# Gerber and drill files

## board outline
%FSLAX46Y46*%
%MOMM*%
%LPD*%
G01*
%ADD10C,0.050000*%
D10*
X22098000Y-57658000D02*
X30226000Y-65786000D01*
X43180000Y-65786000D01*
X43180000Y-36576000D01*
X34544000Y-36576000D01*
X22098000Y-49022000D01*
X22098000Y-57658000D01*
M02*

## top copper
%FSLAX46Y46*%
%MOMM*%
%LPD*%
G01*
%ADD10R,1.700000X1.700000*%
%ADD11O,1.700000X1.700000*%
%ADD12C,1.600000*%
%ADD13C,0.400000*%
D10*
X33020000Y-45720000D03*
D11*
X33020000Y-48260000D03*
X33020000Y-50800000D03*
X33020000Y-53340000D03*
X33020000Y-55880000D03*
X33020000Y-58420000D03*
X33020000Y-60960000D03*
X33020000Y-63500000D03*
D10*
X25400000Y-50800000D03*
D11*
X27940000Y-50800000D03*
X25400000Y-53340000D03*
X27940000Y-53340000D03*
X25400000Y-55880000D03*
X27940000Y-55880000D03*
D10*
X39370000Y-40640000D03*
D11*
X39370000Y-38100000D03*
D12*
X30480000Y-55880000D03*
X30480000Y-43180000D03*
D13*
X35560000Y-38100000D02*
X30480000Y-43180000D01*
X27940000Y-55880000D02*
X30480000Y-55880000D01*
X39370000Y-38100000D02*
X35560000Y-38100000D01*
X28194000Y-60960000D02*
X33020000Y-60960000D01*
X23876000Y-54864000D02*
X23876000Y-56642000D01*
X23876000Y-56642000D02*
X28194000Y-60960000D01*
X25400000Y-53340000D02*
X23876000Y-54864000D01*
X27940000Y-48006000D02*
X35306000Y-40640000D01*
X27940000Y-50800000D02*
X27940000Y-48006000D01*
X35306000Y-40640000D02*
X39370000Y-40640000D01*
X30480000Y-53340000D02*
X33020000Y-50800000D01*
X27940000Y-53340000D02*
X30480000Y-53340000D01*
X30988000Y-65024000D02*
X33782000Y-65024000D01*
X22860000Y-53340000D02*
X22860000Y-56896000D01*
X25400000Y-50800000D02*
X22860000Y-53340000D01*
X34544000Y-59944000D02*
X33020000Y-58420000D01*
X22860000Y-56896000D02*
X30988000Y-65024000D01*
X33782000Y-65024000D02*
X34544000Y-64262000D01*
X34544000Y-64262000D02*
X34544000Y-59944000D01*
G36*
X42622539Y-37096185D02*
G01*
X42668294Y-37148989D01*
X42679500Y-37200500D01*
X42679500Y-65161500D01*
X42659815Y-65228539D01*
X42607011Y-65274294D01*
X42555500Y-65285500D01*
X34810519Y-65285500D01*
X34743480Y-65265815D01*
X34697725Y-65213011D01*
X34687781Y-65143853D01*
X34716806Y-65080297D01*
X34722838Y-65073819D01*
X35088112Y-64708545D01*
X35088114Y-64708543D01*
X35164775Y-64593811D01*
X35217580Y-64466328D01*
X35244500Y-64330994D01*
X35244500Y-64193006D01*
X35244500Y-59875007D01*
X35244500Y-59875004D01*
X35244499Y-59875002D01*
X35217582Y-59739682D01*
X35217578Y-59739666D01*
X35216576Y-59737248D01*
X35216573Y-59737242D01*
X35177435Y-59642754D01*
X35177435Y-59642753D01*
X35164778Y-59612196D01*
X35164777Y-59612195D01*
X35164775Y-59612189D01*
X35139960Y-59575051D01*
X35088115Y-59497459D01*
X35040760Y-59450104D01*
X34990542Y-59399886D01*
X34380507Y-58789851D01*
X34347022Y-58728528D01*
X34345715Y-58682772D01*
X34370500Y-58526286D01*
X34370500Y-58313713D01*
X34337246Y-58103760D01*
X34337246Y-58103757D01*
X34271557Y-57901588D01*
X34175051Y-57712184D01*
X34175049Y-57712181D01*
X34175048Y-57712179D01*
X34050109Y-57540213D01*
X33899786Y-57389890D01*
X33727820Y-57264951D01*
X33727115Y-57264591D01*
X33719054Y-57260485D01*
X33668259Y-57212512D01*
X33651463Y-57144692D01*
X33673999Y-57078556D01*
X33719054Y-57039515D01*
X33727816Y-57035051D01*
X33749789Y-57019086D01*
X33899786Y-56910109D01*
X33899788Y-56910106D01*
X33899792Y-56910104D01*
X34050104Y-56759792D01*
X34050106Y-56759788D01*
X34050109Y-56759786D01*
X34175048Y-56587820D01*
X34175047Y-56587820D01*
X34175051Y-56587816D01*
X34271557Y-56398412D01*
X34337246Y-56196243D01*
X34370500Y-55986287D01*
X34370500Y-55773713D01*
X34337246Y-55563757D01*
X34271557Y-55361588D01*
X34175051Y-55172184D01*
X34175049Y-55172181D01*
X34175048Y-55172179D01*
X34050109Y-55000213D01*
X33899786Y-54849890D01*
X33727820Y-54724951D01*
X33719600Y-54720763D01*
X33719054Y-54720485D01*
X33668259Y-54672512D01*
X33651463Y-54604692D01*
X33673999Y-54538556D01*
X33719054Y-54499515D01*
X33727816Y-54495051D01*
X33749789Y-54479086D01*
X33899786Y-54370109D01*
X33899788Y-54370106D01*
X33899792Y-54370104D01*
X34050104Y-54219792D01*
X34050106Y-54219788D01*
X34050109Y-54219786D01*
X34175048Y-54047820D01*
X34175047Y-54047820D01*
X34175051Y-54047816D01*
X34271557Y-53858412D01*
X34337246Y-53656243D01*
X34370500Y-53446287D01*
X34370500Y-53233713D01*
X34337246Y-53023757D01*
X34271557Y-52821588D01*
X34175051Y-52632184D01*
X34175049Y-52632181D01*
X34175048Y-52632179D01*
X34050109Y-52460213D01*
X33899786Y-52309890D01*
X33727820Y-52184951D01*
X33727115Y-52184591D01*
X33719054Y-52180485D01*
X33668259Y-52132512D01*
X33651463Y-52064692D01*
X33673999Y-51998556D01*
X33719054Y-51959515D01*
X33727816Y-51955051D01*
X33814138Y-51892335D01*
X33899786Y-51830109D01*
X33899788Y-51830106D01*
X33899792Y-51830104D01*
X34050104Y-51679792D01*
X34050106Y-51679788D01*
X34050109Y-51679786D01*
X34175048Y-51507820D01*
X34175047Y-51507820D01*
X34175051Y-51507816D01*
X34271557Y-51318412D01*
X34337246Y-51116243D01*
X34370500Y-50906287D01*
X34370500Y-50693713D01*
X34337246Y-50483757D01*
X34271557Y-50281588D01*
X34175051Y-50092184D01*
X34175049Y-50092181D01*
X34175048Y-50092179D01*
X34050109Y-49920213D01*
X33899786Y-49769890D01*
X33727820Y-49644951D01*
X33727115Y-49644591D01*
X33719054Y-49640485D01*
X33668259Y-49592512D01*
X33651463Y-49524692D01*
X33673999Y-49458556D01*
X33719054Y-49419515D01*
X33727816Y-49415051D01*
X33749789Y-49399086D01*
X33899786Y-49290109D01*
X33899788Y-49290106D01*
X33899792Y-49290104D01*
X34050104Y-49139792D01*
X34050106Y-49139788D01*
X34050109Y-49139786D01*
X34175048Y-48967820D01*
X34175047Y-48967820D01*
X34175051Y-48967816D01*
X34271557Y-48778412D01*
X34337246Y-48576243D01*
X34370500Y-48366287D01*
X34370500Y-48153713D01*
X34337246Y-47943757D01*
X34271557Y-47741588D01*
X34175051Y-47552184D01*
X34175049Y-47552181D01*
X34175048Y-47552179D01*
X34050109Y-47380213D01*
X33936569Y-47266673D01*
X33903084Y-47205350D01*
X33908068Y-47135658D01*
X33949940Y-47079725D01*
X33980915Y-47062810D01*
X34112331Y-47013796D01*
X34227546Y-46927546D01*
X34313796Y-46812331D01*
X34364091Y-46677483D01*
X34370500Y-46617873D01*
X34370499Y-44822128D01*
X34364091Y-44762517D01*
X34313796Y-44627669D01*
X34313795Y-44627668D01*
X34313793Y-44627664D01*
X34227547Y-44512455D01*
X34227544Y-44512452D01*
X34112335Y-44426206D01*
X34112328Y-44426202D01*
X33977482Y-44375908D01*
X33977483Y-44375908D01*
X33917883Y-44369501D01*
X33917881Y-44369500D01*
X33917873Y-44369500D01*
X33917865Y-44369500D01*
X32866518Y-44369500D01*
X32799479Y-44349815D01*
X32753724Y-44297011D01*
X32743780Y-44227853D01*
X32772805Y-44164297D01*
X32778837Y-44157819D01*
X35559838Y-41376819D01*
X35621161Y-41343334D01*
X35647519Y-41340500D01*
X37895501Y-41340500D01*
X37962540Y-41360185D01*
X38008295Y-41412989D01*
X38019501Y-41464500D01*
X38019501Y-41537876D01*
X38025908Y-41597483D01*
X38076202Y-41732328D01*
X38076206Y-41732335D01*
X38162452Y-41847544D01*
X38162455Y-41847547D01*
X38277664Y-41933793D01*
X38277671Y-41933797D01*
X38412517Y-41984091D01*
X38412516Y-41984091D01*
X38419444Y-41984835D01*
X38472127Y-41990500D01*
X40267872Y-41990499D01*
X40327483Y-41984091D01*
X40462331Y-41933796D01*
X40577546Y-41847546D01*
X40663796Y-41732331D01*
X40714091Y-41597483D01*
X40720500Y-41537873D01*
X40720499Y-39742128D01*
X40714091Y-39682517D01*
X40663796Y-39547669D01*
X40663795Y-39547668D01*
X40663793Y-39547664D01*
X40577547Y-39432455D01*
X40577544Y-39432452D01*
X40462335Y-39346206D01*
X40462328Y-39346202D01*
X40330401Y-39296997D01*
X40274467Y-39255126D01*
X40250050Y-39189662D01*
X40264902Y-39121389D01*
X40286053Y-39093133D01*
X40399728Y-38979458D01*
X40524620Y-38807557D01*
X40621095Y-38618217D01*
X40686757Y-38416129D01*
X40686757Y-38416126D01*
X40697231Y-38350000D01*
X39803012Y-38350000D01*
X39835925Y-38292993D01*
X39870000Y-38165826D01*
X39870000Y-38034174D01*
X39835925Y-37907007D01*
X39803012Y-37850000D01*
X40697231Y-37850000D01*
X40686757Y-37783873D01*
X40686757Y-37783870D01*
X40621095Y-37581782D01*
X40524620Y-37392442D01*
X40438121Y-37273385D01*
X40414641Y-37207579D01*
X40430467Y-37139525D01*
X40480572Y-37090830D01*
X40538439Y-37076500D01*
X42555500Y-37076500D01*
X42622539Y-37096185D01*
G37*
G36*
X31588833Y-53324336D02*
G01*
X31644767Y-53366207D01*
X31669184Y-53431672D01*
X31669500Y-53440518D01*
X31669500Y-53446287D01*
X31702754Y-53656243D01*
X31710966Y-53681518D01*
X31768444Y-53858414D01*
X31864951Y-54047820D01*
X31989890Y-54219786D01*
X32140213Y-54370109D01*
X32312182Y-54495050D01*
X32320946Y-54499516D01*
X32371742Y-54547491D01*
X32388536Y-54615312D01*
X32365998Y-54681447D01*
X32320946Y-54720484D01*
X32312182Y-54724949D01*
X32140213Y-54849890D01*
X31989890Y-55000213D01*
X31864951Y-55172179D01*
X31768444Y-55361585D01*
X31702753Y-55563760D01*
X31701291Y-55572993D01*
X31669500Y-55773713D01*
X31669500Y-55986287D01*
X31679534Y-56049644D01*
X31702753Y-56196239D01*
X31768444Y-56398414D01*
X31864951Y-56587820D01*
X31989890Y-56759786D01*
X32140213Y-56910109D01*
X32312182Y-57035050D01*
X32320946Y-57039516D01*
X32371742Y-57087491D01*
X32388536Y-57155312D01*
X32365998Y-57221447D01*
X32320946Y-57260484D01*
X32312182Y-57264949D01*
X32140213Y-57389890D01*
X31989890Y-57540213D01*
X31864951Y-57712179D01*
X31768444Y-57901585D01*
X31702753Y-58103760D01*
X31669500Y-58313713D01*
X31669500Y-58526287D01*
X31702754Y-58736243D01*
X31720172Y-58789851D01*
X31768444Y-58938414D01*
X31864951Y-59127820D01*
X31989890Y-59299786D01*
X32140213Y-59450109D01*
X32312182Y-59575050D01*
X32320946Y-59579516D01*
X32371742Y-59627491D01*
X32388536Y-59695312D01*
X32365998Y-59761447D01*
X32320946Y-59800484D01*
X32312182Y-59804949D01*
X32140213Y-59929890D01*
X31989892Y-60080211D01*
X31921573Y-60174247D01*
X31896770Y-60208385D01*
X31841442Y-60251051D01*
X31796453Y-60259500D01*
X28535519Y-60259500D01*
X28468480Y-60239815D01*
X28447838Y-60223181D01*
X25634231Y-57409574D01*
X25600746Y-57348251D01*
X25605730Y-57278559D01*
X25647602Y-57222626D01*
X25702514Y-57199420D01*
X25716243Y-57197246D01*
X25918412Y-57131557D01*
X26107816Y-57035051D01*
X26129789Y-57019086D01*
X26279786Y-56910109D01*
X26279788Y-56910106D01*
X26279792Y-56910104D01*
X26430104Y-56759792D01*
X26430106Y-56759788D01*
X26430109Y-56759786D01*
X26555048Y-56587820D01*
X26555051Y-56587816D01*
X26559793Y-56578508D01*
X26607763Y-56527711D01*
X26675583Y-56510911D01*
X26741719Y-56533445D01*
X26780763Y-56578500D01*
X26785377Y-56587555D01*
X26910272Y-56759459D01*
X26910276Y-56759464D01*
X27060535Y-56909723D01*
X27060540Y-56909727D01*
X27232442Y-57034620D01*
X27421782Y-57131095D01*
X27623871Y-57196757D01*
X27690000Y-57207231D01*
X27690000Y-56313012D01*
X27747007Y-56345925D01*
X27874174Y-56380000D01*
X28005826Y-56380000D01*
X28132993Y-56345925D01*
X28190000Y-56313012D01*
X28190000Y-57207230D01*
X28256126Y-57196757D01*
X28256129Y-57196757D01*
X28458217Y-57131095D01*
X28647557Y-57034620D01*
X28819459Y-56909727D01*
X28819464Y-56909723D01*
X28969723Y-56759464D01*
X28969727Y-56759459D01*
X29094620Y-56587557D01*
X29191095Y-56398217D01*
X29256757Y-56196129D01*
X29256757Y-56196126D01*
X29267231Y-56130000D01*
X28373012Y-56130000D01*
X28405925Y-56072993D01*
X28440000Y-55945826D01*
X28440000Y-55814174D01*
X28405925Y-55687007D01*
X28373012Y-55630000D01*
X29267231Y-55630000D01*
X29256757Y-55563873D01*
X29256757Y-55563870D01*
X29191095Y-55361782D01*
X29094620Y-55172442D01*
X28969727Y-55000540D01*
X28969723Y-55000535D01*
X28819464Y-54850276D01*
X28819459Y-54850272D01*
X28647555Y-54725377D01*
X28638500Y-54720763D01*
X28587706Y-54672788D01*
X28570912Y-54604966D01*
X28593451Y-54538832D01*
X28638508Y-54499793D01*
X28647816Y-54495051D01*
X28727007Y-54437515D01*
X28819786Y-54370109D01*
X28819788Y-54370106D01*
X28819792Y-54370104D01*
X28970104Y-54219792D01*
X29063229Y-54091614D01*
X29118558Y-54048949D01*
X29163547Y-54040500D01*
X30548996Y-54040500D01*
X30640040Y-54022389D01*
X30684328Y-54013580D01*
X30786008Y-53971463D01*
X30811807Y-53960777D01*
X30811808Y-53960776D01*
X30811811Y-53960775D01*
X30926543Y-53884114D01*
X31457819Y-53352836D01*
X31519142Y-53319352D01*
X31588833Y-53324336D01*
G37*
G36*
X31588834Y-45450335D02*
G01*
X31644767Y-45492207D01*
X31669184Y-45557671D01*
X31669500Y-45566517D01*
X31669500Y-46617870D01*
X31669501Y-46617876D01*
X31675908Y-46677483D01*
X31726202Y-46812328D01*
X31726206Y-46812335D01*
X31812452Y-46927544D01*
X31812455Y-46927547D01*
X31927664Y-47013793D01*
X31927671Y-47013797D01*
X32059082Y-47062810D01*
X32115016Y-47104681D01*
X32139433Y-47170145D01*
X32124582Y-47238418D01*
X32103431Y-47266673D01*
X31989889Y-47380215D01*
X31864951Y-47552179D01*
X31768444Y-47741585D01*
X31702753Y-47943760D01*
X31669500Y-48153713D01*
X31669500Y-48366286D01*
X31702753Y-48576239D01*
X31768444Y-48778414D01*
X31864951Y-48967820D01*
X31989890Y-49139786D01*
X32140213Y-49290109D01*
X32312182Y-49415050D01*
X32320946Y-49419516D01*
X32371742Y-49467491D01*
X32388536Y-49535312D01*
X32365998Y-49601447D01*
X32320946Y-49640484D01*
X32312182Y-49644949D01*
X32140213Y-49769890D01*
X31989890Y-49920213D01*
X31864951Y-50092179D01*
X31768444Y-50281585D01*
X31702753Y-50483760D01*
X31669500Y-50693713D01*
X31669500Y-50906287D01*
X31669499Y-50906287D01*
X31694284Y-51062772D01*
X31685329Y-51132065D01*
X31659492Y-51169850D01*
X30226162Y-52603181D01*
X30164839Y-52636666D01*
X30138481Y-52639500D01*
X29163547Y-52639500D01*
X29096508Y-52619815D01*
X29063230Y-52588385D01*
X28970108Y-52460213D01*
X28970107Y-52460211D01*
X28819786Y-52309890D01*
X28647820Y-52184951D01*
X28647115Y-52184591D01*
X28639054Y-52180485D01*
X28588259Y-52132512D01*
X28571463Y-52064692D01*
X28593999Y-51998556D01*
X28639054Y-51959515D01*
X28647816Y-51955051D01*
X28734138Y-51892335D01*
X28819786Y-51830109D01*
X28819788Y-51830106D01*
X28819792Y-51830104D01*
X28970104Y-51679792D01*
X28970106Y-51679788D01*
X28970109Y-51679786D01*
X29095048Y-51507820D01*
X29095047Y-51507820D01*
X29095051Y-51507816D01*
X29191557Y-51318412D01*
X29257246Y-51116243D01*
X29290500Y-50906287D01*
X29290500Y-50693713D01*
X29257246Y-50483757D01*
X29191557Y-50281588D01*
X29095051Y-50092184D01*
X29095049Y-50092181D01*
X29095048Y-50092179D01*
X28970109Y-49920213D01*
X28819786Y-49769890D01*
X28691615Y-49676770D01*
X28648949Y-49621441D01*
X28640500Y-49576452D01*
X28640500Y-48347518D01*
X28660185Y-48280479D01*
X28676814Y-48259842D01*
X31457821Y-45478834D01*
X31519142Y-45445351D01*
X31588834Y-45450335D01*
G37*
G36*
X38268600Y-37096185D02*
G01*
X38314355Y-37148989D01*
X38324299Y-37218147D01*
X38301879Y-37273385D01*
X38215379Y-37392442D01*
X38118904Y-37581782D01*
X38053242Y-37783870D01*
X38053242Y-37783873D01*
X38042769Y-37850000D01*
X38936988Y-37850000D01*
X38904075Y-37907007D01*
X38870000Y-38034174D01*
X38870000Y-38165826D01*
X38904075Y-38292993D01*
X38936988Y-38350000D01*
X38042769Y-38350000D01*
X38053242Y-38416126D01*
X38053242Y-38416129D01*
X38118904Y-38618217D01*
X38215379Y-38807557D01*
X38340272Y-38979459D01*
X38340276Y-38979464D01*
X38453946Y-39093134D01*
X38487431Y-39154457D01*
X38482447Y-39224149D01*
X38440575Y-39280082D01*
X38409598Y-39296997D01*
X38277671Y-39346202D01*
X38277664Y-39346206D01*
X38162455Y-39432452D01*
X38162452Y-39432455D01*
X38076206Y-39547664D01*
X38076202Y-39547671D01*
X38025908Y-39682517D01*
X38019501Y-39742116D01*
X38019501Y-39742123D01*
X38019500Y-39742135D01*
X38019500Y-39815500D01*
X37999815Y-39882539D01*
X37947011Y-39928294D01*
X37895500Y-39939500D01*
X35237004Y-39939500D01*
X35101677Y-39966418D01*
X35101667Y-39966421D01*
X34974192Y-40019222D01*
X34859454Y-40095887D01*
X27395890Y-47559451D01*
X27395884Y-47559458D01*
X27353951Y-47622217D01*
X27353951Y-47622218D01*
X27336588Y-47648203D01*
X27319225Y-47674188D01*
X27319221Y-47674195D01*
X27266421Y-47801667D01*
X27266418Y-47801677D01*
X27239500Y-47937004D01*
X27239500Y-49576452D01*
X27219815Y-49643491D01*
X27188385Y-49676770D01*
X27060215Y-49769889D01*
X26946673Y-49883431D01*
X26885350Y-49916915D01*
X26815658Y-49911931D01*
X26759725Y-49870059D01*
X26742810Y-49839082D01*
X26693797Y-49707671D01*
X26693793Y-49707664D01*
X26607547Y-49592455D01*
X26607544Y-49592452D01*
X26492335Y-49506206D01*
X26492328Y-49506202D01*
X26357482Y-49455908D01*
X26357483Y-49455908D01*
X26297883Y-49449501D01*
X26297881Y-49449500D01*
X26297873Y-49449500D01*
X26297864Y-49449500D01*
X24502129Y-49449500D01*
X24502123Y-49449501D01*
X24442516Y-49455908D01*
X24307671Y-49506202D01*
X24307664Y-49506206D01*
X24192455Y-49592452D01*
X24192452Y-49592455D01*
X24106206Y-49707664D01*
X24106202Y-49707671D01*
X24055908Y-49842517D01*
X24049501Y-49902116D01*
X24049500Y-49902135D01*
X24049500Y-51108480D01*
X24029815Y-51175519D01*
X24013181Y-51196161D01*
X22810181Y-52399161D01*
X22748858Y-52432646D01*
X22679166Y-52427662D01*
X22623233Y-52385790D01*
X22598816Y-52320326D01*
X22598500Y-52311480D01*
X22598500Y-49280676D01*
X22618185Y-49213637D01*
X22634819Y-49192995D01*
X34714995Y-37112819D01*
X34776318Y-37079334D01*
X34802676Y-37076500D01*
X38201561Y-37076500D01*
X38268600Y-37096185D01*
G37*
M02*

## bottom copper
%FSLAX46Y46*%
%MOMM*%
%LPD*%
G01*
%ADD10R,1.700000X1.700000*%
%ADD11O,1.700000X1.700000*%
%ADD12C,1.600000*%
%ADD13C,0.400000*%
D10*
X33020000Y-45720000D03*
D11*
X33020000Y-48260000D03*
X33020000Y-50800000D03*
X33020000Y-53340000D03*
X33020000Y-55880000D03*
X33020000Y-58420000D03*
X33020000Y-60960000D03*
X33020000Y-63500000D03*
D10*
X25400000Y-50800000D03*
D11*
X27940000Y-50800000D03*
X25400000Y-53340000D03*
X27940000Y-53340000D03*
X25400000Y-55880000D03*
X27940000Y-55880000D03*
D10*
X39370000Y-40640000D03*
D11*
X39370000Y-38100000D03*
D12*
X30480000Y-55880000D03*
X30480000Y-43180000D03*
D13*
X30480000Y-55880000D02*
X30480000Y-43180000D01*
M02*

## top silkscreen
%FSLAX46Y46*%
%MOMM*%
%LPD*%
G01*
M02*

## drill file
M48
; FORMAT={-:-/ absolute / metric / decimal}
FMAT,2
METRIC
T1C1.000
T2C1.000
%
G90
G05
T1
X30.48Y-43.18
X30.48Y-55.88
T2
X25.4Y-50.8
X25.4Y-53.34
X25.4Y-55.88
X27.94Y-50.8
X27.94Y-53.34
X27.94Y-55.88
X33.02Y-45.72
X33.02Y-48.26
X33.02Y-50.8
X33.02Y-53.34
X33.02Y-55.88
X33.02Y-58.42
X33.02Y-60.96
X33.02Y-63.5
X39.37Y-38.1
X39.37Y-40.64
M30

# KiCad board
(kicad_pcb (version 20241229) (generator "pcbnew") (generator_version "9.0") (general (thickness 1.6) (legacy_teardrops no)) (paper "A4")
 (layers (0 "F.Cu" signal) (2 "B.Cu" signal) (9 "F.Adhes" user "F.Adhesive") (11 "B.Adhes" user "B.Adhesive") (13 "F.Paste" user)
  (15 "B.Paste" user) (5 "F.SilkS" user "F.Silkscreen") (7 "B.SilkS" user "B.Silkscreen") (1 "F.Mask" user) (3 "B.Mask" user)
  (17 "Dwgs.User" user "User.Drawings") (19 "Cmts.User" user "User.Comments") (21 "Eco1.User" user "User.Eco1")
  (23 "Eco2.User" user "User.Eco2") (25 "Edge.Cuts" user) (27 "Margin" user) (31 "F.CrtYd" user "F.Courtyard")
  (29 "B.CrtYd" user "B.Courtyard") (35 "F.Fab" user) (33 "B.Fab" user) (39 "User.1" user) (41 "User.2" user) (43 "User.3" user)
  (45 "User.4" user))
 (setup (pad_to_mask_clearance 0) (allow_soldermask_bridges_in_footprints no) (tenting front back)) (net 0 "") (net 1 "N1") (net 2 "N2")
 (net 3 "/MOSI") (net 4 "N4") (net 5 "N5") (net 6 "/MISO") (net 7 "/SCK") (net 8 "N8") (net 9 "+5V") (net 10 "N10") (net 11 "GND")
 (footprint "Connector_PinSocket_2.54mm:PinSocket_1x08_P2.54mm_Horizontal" (layer "B.Cu") (at 33.02 45.72 180)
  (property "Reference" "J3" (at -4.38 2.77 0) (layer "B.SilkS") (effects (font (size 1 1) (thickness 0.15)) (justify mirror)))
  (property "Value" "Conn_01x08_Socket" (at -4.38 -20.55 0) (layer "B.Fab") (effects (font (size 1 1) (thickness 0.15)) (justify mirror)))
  (pad "1" thru_hole rect (at 0 0 180) (size 1.7 1.7) (drill 1) (layers "*.Cu" "*.Mask") (remove_unused_layers no) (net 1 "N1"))
  (pad "2" thru_hole oval (at 0 -2.54 180) (size 1.7 1.7) (drill 1) (layers "*.Cu" "*.Mask") (remove_unused_layers no) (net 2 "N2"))
  (pad "3" thru_hole oval (at 0 -5.08 180) (size 1.7 1.7) (drill 1) (layers "*.Cu" "*.Mask") (remove_unused_layers no) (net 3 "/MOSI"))
  (pad "4" thru_hole oval (at 0 -7.62 180) (size 1.7 1.7) (drill 1) (layers "*.Cu" "*.Mask") (remove_unused_layers no) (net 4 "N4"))
  (pad "5" thru_hole oval (at 0 -10.16 180) (size 1.7 1.7) (drill 1) (layers "*.Cu" "*.Mask") (remove_unused_layers no) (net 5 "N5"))
  (pad "6" thru_hole oval (at 0 -12.7 180) (size 1.7 1.7) (drill 1) (layers "*.Cu" "*.Mask") (remove_unused_layers no) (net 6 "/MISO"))
  (pad "7" thru_hole oval (at 0 -15.24 180) (size 1.7 1.7) (drill 1) (layers "*.Cu" "*.Mask") (remove_unused_layers no) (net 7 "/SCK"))
  (pad "8" thru_hole oval (at 0 -17.78 180) (size 1.7 1.7) (drill 1) (layers "*.Cu" "*.Mask") (remove_unused_layers no) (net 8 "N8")))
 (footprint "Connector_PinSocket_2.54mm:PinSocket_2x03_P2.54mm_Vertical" (layer "B.Cu") (at 25.4 50.8 180)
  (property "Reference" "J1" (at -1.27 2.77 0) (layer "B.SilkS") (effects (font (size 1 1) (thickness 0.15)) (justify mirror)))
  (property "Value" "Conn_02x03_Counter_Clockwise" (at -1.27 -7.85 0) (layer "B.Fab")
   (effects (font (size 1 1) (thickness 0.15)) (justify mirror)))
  (pad "1" thru_hole rect (at 0 0 180) (size 1.7 1.7) (drill 1) (layers "*.Cu" "*.Mask") (remove_unused_layers no) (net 6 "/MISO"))
  (pad "2" thru_hole oval (at -2.54 0 180) (size 1.7 1.7) (drill 1) (layers "*.Cu" "*.Mask") (remove_unused_layers no) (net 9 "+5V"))
  (pad "3" thru_hole oval (at 0 -2.54 180) (size 1.7 1.7) (drill 1) (layers "*.Cu" "*.Mask") (remove_unused_layers no) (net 7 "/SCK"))
  (pad "4" thru_hole oval (at -2.54 -2.54 180) (size 1.7 1.7) (drill 1) (layers "*.Cu" "*.Mask") (remove_unused_layers no) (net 3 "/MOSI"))
  (pad "5" thru_hole oval (at 0 -5.08 180) (size 1.7 1.7) (drill 1) (layers "*.Cu" "*.Mask") (remove_unused_layers no) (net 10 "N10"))
  (pad "6" thru_hole oval (at -2.54 -5.08 180) (size 1.7 1.7) (drill 1) (layers "*.Cu" "*.Mask") (remove_unused_layers no) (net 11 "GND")))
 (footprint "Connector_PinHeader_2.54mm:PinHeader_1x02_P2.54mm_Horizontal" (layer "B.Cu") (at 39.37 40.64)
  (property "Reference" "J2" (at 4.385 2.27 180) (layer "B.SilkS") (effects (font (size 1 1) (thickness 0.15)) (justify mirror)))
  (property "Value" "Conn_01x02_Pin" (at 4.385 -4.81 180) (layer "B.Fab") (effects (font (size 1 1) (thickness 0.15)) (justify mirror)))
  (pad "1" thru_hole rect (at 0 0) (size 1.7 1.7) (drill 1) (layers "*.Cu" "*.Mask") (remove_unused_layers no) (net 9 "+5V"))
  (pad "2" thru_hole oval (at 0 -2.54) (size 1.7 1.7) (drill 1) (layers "*.Cu" "*.Mask") (remove_unused_layers no) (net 11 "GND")))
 (gr_poly
  (pts (xy 22.098 57.658) (xy 30.226 65.786) (xy 43.18 65.786) (xy 43.18 36.576) (xy 34.544 36.576) (xy 22.098 49.022))
  (stroke (width 0.05) (type solid)) (fill no) (layer "Edge.Cuts"))
 (segment (start 35.56 38.1) (end 30.48 43.18) (width 0.4) (layer "F.Cu") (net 11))
 (segment (start 27.94 55.88) (end 30.48 55.88) (width 0.4) (layer "F.Cu") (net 11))
 (segment (start 39.37 38.1) (end 35.56 38.1) (width 0.4) (layer "F.Cu") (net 11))
 (via (at 30.48 55.88) (size 1.6) (drill 1) (layers "F.Cu" "B.Cu") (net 11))
 (via (at 30.48 43.18) (size 1.6) (drill 1) (layers "F.Cu" "B.Cu") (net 11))
 (segment (start 30.48 55.88) (end 30.48 43.18) (width 0.4) (layer "B.Cu") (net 11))
 (segment (start 28.194 60.96) (end 33.02 60.96) (width 0.4) (layer "F.Cu") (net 7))
 (segment (start 23.876 54.864) (end 23.876 56.642) (width 0.4) (layer "F.Cu") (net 7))
 (segment (start 23.876 56.642) (end 28.194 60.96) (width 0.4) (layer "F.Cu") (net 7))
 (segment (start 25.4 53.34) (end 23.876 54.864) (width 0.4) (layer "F.Cu") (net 7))
 (segment (start 27.94 48.006) (end 35.306 40.64) (width 0.4) (layer "F.Cu") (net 9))
 (segment (start 27.94 50.8) (end 27.94 48.006) (width 0.4) (layer "F.Cu") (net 9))
 (segment (start 35.306 40.64) (end 39.37 40.64) (width 0.4) (layer "F.Cu") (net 9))
 (segment (start 30.48 53.34) (end 33.02 50.8) (width 0.4) (layer "F.Cu") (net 3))
 (segment (start 27.94 53.34) (end 30.48 53.34) (width 0.4) (layer "F.Cu") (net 3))
 (segment (start 30.988 65.024) (end 33.782 65.024) (width 0.4) (layer "F.Cu") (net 6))
 (segment (start 22.86 53.34) (end 22.86 56.896) (width 0.4) (layer "F.Cu") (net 6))
 (segment (start 25.4 50.8) (end 22.86 53.34) (width 0.4) (layer "F.Cu") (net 6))
 (segment (start 34.544 59.944) (end 33.02 58.42) (width 0.4) (layer "F.Cu") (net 6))
 (segment (start 22.86 56.896) (end 30.988 65.024) (width 0.4) (layer "F.Cu") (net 6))
 (segment (start 33.782 65.024) (end 34.544 64.262) (width 0.4) (layer "F.Cu") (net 6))
 (segment (start 34.544 64.262) (end 34.544 59.944) (width 0.4) (layer "F.Cu") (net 6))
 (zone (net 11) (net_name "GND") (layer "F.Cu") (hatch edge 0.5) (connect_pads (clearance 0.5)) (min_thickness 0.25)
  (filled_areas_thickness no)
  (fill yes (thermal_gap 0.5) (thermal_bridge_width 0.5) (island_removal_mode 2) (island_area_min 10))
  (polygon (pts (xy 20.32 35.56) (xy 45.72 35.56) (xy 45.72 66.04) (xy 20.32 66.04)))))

